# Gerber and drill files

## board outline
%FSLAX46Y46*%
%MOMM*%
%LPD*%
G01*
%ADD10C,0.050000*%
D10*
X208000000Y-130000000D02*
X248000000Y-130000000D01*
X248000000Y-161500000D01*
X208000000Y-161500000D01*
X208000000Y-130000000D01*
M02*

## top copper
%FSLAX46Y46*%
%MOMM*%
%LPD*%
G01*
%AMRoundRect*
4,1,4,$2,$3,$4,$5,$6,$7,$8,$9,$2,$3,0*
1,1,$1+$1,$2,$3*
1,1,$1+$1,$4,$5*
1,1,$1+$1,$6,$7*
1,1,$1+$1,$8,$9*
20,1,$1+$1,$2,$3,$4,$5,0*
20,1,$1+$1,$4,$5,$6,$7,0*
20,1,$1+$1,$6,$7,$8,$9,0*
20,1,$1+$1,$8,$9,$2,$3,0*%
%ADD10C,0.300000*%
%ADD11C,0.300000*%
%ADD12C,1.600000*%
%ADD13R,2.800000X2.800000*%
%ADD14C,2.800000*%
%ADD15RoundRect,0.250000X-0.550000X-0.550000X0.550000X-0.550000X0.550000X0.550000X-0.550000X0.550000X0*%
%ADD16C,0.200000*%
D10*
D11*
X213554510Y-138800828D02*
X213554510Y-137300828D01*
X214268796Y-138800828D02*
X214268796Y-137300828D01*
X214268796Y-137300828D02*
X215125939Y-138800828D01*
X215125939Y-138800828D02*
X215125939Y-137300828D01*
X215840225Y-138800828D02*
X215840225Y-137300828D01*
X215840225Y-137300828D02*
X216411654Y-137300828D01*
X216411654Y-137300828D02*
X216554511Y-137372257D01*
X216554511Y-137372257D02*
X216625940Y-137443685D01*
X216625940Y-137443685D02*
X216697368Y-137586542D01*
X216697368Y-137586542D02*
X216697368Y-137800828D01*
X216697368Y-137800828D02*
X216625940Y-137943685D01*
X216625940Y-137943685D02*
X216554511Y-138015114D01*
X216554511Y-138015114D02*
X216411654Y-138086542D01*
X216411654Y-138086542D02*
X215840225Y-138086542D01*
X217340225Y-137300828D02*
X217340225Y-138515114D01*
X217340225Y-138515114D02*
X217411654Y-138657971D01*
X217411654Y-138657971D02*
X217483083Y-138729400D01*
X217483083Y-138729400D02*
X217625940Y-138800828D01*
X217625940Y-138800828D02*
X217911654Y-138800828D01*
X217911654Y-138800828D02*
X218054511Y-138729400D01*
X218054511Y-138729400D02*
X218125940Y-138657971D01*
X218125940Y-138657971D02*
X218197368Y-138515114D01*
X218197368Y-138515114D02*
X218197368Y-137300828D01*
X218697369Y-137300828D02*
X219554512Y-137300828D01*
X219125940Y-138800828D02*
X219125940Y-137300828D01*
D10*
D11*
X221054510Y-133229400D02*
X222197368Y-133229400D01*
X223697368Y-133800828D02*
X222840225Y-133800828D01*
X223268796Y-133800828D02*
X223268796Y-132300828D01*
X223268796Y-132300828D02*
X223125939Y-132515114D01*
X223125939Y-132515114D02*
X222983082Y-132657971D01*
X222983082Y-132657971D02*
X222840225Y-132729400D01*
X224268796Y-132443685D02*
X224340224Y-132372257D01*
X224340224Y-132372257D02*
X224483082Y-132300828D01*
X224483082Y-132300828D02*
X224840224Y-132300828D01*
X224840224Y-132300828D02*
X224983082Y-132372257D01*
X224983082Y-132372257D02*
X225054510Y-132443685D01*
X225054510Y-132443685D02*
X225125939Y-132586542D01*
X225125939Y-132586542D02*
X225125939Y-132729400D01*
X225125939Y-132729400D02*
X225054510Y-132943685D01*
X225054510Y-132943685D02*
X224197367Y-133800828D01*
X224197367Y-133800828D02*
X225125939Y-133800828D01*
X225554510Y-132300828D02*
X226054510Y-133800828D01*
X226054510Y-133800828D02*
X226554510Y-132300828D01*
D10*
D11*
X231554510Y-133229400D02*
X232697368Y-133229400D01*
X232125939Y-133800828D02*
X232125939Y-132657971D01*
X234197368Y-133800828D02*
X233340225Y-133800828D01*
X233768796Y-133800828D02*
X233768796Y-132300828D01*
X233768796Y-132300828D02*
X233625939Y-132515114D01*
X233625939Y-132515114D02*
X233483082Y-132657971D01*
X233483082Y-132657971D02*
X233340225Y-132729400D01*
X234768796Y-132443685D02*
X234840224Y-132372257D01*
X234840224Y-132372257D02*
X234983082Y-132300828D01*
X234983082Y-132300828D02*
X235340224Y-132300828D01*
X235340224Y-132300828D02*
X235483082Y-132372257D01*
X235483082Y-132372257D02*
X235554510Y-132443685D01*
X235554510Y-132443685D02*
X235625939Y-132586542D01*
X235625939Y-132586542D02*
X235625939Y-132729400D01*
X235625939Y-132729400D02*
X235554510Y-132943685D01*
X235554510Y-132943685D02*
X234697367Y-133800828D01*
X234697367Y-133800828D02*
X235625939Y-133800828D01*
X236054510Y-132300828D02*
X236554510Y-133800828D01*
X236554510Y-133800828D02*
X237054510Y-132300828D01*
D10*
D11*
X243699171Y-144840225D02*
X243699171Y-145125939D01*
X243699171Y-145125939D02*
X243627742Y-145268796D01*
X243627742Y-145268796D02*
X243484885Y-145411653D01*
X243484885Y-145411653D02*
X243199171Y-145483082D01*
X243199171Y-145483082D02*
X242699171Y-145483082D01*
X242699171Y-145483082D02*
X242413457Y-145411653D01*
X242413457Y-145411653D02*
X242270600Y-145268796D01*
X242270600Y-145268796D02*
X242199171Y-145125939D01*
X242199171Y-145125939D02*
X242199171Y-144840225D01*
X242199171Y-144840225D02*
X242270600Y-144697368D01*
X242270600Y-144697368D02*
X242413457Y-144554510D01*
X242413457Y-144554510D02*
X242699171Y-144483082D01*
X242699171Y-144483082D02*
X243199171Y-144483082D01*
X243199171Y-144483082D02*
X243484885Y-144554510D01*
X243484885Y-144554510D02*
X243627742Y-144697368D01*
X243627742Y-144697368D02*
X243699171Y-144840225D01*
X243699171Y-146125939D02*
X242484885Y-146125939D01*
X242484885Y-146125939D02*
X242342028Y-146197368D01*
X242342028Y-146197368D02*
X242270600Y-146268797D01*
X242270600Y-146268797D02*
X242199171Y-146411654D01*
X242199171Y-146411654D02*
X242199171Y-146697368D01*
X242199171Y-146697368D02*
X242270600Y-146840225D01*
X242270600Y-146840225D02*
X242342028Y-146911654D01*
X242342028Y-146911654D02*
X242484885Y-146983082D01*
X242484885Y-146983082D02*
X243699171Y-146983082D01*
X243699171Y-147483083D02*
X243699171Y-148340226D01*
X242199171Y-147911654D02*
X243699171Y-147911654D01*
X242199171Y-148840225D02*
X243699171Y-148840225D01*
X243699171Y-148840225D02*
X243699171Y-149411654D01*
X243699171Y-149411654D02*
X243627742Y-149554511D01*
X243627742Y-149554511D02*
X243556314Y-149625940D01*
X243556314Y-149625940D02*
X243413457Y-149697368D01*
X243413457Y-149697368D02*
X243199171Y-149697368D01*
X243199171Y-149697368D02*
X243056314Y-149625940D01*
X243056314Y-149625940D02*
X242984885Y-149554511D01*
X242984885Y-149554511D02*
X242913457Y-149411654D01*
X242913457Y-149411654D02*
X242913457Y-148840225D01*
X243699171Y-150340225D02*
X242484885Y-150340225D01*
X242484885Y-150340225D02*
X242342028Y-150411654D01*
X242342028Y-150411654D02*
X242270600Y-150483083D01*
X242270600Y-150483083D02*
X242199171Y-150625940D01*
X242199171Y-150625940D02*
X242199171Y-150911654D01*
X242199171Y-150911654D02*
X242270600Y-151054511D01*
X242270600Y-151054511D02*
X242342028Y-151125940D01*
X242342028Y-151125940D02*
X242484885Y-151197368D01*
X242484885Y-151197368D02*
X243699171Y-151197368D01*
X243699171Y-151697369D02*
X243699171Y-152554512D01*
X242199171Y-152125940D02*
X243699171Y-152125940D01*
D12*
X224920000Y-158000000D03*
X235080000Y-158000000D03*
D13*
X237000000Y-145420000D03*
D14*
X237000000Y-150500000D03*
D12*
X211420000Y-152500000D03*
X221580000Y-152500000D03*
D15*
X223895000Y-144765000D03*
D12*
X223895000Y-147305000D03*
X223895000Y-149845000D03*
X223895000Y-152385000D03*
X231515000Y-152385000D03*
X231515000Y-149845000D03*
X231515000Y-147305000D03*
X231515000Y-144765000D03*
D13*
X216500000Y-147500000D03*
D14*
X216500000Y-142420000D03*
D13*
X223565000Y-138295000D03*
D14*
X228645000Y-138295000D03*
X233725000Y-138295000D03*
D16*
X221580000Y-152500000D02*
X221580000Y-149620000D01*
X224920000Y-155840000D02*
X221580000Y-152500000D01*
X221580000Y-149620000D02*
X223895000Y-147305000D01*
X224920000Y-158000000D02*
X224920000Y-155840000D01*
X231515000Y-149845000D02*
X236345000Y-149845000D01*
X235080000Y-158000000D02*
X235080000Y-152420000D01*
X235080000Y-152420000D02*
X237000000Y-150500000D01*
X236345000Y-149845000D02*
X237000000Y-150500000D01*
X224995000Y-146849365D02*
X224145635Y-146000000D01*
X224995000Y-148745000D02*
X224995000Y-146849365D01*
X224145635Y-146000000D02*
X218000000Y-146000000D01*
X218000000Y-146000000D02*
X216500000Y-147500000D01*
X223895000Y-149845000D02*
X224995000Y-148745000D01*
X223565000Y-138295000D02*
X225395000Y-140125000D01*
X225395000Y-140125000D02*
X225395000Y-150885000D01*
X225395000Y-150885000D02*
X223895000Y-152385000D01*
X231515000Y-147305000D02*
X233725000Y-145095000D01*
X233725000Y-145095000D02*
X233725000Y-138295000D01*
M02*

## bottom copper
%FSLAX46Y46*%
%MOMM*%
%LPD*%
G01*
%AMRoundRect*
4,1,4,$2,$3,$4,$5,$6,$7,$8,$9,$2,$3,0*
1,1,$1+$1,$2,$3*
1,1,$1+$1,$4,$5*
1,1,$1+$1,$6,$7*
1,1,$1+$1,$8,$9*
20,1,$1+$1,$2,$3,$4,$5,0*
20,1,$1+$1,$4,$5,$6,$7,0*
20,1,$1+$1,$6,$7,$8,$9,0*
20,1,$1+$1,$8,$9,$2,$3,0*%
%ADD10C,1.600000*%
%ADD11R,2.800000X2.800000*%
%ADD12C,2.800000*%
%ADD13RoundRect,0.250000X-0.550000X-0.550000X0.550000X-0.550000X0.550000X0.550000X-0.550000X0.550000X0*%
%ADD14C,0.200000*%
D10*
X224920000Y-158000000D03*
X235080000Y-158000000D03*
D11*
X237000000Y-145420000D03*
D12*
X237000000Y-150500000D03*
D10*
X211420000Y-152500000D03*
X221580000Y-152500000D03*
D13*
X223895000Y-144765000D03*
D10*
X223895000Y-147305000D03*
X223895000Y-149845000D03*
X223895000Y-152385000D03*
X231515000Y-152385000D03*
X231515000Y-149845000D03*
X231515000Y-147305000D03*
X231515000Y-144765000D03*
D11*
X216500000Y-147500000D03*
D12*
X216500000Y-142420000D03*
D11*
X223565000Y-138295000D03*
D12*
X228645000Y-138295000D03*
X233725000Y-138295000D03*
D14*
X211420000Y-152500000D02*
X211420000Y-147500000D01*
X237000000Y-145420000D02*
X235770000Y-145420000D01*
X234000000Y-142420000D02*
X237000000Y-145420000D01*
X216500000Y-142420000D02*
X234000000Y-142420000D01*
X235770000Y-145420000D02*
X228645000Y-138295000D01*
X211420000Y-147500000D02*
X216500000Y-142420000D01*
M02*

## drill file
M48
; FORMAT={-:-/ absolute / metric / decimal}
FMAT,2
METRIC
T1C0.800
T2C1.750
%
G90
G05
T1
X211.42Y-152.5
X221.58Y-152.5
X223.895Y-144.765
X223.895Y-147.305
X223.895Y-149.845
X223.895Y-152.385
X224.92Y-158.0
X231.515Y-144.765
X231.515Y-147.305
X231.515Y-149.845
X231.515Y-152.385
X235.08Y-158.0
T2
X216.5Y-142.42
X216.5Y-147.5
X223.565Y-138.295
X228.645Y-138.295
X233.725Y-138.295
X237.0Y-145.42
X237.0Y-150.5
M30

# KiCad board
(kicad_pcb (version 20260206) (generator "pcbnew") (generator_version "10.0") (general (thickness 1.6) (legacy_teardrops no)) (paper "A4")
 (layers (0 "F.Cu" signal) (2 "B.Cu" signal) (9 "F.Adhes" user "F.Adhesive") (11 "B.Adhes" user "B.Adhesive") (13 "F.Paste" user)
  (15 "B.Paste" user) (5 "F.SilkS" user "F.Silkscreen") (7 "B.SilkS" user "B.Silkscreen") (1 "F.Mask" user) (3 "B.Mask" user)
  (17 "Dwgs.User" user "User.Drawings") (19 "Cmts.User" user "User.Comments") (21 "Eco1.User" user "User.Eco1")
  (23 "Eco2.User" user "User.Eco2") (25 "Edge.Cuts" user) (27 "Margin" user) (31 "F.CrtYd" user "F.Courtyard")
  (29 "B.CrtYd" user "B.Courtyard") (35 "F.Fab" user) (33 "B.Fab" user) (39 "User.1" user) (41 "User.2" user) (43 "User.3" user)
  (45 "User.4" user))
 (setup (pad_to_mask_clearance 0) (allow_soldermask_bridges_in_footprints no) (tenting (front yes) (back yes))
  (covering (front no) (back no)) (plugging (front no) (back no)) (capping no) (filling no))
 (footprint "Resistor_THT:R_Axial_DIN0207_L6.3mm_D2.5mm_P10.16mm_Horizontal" (layer "F.Cu") (at 224.92 158)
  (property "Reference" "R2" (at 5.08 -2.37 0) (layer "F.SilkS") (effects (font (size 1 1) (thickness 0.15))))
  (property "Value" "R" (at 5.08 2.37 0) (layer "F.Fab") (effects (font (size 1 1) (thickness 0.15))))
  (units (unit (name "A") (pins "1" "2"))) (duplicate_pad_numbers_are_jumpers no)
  (pad "1" thru_hole circle (at 0 0) (size 1.6 1.6) (drill 0.8) (layers "*.Cu" "*.Mask") (remove_unused_layers no) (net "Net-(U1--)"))
  (pad "2" thru_hole circle (at 10.16 0) (size 1.6 1.6) (drill 0.8) (layers "*.Cu" "*.Mask") (remove_unused_layers no)
   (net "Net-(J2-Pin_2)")))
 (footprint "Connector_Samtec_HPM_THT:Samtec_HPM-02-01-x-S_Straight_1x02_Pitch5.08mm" (layer "F.Cu") (at 237 145.42)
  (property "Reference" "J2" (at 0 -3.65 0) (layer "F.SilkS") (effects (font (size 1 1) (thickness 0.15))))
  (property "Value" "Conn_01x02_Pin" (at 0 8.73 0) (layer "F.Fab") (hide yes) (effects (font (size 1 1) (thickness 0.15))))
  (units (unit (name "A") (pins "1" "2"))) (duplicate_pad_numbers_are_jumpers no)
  (pad "1" thru_hole rect (at 0 0) (size 2.8 2.8) (drill 1.75) (layers "*.Cu" "*.Mask") (remove_unused_layers no) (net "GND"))
  (pad "2" thru_hole circle (at 0 5.08) (size 2.8 2.8) (drill 1.75) (layers "*.Cu" "*.Mask") (remove_unused_layers no)
   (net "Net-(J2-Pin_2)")))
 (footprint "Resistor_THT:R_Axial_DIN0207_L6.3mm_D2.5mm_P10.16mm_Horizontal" (layer "F.Cu") (at 211.42 152.5)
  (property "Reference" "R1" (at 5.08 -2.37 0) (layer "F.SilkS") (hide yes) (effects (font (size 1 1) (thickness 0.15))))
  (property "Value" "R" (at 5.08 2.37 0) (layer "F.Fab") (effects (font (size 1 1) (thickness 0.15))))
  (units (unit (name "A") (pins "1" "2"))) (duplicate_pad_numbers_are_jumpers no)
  (pad "1" thru_hole circle (at 0 0) (size 1.6 1.6) (drill 0.8) (layers "*.Cu" "*.Mask") (remove_unused_layers no) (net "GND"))
  (pad "2" thru_hole circle (at 10.16 0) (size 1.6 1.6) (drill 0.8) (layers "*.Cu" "*.Mask") (remove_unused_layers no) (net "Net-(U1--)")))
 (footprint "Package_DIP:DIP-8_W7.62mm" (layer "F.Cu") (at 223.895 144.765)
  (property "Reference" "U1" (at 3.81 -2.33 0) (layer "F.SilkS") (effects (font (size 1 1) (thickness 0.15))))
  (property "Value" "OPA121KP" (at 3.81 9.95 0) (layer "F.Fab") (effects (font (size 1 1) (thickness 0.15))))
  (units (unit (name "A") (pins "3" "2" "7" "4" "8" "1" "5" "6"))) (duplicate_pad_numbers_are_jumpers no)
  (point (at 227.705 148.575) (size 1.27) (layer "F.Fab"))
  (pad "1" thru_hole roundrect (at 0 0) (size 1.6 1.6) (drill 0.8) (layers "*.Cu" "*.Mask") (remove_unused_layers no)
   (roundrect_rratio 0.15625) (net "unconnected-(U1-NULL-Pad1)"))
  (pad "2" thru_hole circle (at 0 2.54) (size 1.6 1.6) (drill 0.8) (layers "*.Cu" "*.Mask") (remove_unused_layers no) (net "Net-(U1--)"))
  (pad "3" thru_hole circle (at 0 5.08) (size 1.6 1.6) (drill 0.8) (layers "*.Cu" "*.Mask") (remove_unused_layers no) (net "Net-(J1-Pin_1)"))
  (pad "4" thru_hole circle (at 0 7.62) (size 1.6 1.6) (drill 0.8) (layers "*.Cu" "*.Mask") (remove_unused_layers no) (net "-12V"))
  (pad "5" thru_hole circle (at 7.62 7.62) (size 1.6 1.6) (drill 0.8) (layers "*.Cu" "*.Mask") (remove_unused_layers no)
   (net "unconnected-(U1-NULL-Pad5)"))
  (pad "6" thru_hole circle (at 7.62 5.08) (size 1.6 1.6) (drill 0.8) (layers "*.Cu" "*.Mask") (remove_unused_layers no)
   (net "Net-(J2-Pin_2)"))
  (pad "7" thru_hole circle (at 7.62 2.54) (size 1.6 1.6) (drill 0.8) (layers "*.Cu" "*.Mask") (remove_unused_layers no) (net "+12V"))
  (pad "8" thru_hole circle (at 7.62 0) (size 1.6 1.6) (drill 0.8) (layers "*.Cu" "*.Mask") (remove_unused_layers no)
   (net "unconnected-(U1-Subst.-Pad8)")))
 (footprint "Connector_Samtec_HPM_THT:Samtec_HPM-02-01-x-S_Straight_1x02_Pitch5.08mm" (layer "F.Cu") (at 216.5 147.5 180)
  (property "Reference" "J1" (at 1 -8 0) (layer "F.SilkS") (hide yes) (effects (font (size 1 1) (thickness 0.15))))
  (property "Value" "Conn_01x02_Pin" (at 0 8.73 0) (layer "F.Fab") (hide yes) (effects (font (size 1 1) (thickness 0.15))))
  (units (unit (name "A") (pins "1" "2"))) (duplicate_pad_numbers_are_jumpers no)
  (pad "1" thru_hole rect (at 0 0 180) (size 2.8 2.8) (drill 1.75) (layers "*.Cu" "*.Mask") (remove_unused_layers no) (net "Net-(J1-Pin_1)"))
  (pad "2" thru_hole circle (at 0 5.08 180) (size 2.8 2.8) (drill 1.75) (layers "*.Cu" "*.Mask") (remove_unused_layers no) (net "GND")))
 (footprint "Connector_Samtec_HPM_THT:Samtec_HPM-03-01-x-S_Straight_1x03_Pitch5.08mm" (layer "F.Cu") (at 223.565 138.295 90)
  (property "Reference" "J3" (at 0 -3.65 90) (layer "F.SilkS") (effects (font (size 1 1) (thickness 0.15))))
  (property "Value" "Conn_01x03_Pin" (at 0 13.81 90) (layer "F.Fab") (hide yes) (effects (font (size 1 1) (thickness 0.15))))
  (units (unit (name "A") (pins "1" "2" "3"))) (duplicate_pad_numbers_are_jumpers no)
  (pad "1" thru_hole rect (at 0 0 90) (size 2.8 2.8) (drill 1.75) (layers "*.Cu" "*.Mask") (remove_unused_layers no) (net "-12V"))
  (pad "2" thru_hole circle (at 0 5.08 90) (size 2.8 2.8) (drill 1.75) (layers "*.Cu" "*.Mask") (remove_unused_layers no) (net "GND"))
  (pad "3" thru_hole circle (at 0 10.16 90) (size 2.8 2.8) (drill 1.75) (layers "*.Cu" "*.Mask") (remove_unused_layers no) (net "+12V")))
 (gr_rect (start 208 130) (end 248 161.5) (stroke (width 0.05) (type default)) (fill no) (layer "Edge.Cuts"))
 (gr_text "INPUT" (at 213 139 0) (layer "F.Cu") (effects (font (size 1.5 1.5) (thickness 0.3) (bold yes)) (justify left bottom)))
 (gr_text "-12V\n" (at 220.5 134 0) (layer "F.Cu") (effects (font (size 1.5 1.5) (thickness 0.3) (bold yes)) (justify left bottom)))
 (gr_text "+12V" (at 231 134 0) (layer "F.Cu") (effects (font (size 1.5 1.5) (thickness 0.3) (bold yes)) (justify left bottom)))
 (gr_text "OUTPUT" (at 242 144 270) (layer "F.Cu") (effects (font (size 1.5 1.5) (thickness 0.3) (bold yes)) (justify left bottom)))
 (segment (start 221.58 152.5) (end 221.58 149.62) (width 0.2) (layer "F.Cu") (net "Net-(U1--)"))
 (segment (start 224.92 155.84) (end 221.58 152.5) (width 0.2) (layer "F.Cu") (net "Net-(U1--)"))
 (segment (start 221.58 149.62) (end 223.895 147.305) (width 0.2) (layer "F.Cu") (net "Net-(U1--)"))
 (segment (start 224.92 158) (end 224.92 155.84) (width 0.2) (layer "F.Cu") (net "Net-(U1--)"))
 (segment (start 231.515 149.845) (end 236.345 149.845) (width 0.2) (layer "F.Cu") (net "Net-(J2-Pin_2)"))
 (segment (start 235.08 158) (end 235.08 152.42) (width 0.2) (layer "F.Cu") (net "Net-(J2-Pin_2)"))
 (segment (start 235.08 152.42) (end 237 150.5) (width 0.2) (layer "F.Cu") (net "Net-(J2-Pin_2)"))
 (segment (start 236.345 149.845) (end 237 150.5) (width 0.2) (layer "F.Cu") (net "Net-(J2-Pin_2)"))
 (segment (start 211.42 152.5) (end 211.42 147.5) (width 0.2) (layer "B.Cu") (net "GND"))
 (segment (start 237 145.42) (end 235.77 145.42) (width 0.2) (layer "B.Cu") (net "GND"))
 (segment (start 234 142.42) (end 237 145.42) (width 0.2) (layer "B.Cu") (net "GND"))
 (segment (start 216.5 142.42) (end 234 142.42) (width 0.2) (layer "B.Cu") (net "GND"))
 (segment (start 235.77 145.42) (end 228.645 138.295) (width 0.2) (layer "B.Cu") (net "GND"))
 (segment (start 211.42 147.5) (end 216.5 142.42) (width 0.2) (layer "B.Cu") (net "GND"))
 (segment (start 224.995 146.849365) (end 224.145635 146) (width 0.2) (layer "F.Cu") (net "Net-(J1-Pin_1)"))
 (segment (start 224.995 148.745) (end 224.995 146.849365) (width 0.2) (layer "F.Cu") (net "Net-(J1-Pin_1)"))
 (segment (start 224.145635 146) (end 218 146) (width 0.2) (layer "F.Cu") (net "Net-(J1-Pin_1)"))
 (segment (start 218 146) (end 216.5 147.5) (width 0.2) (layer "F.Cu") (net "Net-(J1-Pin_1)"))
 (segment (start 223.895 149.845) (end 224.995 148.745) (width 0.2) (layer "F.Cu") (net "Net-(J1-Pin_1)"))
 (segment (start 223.565 138.295) (end 225.395 140.125) (width 0.2) (layer "F.Cu") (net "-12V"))
 (segment (start 225.395 140.125) (end 225.395 150.885) (width 0.2) (layer "F.Cu") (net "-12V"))
 (segment (start 225.395 150.885) (end 223.895 152.385) (width 0.2) (layer "F.Cu") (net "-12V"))
 (segment (start 231.515 147.305) (end 233.725 145.095) (width 0.2) (layer "F.Cu") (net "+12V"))
 (segment (start 233.725 145.095) (end 233.725 138.295) (width 0.2) (layer "F.Cu") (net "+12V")))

